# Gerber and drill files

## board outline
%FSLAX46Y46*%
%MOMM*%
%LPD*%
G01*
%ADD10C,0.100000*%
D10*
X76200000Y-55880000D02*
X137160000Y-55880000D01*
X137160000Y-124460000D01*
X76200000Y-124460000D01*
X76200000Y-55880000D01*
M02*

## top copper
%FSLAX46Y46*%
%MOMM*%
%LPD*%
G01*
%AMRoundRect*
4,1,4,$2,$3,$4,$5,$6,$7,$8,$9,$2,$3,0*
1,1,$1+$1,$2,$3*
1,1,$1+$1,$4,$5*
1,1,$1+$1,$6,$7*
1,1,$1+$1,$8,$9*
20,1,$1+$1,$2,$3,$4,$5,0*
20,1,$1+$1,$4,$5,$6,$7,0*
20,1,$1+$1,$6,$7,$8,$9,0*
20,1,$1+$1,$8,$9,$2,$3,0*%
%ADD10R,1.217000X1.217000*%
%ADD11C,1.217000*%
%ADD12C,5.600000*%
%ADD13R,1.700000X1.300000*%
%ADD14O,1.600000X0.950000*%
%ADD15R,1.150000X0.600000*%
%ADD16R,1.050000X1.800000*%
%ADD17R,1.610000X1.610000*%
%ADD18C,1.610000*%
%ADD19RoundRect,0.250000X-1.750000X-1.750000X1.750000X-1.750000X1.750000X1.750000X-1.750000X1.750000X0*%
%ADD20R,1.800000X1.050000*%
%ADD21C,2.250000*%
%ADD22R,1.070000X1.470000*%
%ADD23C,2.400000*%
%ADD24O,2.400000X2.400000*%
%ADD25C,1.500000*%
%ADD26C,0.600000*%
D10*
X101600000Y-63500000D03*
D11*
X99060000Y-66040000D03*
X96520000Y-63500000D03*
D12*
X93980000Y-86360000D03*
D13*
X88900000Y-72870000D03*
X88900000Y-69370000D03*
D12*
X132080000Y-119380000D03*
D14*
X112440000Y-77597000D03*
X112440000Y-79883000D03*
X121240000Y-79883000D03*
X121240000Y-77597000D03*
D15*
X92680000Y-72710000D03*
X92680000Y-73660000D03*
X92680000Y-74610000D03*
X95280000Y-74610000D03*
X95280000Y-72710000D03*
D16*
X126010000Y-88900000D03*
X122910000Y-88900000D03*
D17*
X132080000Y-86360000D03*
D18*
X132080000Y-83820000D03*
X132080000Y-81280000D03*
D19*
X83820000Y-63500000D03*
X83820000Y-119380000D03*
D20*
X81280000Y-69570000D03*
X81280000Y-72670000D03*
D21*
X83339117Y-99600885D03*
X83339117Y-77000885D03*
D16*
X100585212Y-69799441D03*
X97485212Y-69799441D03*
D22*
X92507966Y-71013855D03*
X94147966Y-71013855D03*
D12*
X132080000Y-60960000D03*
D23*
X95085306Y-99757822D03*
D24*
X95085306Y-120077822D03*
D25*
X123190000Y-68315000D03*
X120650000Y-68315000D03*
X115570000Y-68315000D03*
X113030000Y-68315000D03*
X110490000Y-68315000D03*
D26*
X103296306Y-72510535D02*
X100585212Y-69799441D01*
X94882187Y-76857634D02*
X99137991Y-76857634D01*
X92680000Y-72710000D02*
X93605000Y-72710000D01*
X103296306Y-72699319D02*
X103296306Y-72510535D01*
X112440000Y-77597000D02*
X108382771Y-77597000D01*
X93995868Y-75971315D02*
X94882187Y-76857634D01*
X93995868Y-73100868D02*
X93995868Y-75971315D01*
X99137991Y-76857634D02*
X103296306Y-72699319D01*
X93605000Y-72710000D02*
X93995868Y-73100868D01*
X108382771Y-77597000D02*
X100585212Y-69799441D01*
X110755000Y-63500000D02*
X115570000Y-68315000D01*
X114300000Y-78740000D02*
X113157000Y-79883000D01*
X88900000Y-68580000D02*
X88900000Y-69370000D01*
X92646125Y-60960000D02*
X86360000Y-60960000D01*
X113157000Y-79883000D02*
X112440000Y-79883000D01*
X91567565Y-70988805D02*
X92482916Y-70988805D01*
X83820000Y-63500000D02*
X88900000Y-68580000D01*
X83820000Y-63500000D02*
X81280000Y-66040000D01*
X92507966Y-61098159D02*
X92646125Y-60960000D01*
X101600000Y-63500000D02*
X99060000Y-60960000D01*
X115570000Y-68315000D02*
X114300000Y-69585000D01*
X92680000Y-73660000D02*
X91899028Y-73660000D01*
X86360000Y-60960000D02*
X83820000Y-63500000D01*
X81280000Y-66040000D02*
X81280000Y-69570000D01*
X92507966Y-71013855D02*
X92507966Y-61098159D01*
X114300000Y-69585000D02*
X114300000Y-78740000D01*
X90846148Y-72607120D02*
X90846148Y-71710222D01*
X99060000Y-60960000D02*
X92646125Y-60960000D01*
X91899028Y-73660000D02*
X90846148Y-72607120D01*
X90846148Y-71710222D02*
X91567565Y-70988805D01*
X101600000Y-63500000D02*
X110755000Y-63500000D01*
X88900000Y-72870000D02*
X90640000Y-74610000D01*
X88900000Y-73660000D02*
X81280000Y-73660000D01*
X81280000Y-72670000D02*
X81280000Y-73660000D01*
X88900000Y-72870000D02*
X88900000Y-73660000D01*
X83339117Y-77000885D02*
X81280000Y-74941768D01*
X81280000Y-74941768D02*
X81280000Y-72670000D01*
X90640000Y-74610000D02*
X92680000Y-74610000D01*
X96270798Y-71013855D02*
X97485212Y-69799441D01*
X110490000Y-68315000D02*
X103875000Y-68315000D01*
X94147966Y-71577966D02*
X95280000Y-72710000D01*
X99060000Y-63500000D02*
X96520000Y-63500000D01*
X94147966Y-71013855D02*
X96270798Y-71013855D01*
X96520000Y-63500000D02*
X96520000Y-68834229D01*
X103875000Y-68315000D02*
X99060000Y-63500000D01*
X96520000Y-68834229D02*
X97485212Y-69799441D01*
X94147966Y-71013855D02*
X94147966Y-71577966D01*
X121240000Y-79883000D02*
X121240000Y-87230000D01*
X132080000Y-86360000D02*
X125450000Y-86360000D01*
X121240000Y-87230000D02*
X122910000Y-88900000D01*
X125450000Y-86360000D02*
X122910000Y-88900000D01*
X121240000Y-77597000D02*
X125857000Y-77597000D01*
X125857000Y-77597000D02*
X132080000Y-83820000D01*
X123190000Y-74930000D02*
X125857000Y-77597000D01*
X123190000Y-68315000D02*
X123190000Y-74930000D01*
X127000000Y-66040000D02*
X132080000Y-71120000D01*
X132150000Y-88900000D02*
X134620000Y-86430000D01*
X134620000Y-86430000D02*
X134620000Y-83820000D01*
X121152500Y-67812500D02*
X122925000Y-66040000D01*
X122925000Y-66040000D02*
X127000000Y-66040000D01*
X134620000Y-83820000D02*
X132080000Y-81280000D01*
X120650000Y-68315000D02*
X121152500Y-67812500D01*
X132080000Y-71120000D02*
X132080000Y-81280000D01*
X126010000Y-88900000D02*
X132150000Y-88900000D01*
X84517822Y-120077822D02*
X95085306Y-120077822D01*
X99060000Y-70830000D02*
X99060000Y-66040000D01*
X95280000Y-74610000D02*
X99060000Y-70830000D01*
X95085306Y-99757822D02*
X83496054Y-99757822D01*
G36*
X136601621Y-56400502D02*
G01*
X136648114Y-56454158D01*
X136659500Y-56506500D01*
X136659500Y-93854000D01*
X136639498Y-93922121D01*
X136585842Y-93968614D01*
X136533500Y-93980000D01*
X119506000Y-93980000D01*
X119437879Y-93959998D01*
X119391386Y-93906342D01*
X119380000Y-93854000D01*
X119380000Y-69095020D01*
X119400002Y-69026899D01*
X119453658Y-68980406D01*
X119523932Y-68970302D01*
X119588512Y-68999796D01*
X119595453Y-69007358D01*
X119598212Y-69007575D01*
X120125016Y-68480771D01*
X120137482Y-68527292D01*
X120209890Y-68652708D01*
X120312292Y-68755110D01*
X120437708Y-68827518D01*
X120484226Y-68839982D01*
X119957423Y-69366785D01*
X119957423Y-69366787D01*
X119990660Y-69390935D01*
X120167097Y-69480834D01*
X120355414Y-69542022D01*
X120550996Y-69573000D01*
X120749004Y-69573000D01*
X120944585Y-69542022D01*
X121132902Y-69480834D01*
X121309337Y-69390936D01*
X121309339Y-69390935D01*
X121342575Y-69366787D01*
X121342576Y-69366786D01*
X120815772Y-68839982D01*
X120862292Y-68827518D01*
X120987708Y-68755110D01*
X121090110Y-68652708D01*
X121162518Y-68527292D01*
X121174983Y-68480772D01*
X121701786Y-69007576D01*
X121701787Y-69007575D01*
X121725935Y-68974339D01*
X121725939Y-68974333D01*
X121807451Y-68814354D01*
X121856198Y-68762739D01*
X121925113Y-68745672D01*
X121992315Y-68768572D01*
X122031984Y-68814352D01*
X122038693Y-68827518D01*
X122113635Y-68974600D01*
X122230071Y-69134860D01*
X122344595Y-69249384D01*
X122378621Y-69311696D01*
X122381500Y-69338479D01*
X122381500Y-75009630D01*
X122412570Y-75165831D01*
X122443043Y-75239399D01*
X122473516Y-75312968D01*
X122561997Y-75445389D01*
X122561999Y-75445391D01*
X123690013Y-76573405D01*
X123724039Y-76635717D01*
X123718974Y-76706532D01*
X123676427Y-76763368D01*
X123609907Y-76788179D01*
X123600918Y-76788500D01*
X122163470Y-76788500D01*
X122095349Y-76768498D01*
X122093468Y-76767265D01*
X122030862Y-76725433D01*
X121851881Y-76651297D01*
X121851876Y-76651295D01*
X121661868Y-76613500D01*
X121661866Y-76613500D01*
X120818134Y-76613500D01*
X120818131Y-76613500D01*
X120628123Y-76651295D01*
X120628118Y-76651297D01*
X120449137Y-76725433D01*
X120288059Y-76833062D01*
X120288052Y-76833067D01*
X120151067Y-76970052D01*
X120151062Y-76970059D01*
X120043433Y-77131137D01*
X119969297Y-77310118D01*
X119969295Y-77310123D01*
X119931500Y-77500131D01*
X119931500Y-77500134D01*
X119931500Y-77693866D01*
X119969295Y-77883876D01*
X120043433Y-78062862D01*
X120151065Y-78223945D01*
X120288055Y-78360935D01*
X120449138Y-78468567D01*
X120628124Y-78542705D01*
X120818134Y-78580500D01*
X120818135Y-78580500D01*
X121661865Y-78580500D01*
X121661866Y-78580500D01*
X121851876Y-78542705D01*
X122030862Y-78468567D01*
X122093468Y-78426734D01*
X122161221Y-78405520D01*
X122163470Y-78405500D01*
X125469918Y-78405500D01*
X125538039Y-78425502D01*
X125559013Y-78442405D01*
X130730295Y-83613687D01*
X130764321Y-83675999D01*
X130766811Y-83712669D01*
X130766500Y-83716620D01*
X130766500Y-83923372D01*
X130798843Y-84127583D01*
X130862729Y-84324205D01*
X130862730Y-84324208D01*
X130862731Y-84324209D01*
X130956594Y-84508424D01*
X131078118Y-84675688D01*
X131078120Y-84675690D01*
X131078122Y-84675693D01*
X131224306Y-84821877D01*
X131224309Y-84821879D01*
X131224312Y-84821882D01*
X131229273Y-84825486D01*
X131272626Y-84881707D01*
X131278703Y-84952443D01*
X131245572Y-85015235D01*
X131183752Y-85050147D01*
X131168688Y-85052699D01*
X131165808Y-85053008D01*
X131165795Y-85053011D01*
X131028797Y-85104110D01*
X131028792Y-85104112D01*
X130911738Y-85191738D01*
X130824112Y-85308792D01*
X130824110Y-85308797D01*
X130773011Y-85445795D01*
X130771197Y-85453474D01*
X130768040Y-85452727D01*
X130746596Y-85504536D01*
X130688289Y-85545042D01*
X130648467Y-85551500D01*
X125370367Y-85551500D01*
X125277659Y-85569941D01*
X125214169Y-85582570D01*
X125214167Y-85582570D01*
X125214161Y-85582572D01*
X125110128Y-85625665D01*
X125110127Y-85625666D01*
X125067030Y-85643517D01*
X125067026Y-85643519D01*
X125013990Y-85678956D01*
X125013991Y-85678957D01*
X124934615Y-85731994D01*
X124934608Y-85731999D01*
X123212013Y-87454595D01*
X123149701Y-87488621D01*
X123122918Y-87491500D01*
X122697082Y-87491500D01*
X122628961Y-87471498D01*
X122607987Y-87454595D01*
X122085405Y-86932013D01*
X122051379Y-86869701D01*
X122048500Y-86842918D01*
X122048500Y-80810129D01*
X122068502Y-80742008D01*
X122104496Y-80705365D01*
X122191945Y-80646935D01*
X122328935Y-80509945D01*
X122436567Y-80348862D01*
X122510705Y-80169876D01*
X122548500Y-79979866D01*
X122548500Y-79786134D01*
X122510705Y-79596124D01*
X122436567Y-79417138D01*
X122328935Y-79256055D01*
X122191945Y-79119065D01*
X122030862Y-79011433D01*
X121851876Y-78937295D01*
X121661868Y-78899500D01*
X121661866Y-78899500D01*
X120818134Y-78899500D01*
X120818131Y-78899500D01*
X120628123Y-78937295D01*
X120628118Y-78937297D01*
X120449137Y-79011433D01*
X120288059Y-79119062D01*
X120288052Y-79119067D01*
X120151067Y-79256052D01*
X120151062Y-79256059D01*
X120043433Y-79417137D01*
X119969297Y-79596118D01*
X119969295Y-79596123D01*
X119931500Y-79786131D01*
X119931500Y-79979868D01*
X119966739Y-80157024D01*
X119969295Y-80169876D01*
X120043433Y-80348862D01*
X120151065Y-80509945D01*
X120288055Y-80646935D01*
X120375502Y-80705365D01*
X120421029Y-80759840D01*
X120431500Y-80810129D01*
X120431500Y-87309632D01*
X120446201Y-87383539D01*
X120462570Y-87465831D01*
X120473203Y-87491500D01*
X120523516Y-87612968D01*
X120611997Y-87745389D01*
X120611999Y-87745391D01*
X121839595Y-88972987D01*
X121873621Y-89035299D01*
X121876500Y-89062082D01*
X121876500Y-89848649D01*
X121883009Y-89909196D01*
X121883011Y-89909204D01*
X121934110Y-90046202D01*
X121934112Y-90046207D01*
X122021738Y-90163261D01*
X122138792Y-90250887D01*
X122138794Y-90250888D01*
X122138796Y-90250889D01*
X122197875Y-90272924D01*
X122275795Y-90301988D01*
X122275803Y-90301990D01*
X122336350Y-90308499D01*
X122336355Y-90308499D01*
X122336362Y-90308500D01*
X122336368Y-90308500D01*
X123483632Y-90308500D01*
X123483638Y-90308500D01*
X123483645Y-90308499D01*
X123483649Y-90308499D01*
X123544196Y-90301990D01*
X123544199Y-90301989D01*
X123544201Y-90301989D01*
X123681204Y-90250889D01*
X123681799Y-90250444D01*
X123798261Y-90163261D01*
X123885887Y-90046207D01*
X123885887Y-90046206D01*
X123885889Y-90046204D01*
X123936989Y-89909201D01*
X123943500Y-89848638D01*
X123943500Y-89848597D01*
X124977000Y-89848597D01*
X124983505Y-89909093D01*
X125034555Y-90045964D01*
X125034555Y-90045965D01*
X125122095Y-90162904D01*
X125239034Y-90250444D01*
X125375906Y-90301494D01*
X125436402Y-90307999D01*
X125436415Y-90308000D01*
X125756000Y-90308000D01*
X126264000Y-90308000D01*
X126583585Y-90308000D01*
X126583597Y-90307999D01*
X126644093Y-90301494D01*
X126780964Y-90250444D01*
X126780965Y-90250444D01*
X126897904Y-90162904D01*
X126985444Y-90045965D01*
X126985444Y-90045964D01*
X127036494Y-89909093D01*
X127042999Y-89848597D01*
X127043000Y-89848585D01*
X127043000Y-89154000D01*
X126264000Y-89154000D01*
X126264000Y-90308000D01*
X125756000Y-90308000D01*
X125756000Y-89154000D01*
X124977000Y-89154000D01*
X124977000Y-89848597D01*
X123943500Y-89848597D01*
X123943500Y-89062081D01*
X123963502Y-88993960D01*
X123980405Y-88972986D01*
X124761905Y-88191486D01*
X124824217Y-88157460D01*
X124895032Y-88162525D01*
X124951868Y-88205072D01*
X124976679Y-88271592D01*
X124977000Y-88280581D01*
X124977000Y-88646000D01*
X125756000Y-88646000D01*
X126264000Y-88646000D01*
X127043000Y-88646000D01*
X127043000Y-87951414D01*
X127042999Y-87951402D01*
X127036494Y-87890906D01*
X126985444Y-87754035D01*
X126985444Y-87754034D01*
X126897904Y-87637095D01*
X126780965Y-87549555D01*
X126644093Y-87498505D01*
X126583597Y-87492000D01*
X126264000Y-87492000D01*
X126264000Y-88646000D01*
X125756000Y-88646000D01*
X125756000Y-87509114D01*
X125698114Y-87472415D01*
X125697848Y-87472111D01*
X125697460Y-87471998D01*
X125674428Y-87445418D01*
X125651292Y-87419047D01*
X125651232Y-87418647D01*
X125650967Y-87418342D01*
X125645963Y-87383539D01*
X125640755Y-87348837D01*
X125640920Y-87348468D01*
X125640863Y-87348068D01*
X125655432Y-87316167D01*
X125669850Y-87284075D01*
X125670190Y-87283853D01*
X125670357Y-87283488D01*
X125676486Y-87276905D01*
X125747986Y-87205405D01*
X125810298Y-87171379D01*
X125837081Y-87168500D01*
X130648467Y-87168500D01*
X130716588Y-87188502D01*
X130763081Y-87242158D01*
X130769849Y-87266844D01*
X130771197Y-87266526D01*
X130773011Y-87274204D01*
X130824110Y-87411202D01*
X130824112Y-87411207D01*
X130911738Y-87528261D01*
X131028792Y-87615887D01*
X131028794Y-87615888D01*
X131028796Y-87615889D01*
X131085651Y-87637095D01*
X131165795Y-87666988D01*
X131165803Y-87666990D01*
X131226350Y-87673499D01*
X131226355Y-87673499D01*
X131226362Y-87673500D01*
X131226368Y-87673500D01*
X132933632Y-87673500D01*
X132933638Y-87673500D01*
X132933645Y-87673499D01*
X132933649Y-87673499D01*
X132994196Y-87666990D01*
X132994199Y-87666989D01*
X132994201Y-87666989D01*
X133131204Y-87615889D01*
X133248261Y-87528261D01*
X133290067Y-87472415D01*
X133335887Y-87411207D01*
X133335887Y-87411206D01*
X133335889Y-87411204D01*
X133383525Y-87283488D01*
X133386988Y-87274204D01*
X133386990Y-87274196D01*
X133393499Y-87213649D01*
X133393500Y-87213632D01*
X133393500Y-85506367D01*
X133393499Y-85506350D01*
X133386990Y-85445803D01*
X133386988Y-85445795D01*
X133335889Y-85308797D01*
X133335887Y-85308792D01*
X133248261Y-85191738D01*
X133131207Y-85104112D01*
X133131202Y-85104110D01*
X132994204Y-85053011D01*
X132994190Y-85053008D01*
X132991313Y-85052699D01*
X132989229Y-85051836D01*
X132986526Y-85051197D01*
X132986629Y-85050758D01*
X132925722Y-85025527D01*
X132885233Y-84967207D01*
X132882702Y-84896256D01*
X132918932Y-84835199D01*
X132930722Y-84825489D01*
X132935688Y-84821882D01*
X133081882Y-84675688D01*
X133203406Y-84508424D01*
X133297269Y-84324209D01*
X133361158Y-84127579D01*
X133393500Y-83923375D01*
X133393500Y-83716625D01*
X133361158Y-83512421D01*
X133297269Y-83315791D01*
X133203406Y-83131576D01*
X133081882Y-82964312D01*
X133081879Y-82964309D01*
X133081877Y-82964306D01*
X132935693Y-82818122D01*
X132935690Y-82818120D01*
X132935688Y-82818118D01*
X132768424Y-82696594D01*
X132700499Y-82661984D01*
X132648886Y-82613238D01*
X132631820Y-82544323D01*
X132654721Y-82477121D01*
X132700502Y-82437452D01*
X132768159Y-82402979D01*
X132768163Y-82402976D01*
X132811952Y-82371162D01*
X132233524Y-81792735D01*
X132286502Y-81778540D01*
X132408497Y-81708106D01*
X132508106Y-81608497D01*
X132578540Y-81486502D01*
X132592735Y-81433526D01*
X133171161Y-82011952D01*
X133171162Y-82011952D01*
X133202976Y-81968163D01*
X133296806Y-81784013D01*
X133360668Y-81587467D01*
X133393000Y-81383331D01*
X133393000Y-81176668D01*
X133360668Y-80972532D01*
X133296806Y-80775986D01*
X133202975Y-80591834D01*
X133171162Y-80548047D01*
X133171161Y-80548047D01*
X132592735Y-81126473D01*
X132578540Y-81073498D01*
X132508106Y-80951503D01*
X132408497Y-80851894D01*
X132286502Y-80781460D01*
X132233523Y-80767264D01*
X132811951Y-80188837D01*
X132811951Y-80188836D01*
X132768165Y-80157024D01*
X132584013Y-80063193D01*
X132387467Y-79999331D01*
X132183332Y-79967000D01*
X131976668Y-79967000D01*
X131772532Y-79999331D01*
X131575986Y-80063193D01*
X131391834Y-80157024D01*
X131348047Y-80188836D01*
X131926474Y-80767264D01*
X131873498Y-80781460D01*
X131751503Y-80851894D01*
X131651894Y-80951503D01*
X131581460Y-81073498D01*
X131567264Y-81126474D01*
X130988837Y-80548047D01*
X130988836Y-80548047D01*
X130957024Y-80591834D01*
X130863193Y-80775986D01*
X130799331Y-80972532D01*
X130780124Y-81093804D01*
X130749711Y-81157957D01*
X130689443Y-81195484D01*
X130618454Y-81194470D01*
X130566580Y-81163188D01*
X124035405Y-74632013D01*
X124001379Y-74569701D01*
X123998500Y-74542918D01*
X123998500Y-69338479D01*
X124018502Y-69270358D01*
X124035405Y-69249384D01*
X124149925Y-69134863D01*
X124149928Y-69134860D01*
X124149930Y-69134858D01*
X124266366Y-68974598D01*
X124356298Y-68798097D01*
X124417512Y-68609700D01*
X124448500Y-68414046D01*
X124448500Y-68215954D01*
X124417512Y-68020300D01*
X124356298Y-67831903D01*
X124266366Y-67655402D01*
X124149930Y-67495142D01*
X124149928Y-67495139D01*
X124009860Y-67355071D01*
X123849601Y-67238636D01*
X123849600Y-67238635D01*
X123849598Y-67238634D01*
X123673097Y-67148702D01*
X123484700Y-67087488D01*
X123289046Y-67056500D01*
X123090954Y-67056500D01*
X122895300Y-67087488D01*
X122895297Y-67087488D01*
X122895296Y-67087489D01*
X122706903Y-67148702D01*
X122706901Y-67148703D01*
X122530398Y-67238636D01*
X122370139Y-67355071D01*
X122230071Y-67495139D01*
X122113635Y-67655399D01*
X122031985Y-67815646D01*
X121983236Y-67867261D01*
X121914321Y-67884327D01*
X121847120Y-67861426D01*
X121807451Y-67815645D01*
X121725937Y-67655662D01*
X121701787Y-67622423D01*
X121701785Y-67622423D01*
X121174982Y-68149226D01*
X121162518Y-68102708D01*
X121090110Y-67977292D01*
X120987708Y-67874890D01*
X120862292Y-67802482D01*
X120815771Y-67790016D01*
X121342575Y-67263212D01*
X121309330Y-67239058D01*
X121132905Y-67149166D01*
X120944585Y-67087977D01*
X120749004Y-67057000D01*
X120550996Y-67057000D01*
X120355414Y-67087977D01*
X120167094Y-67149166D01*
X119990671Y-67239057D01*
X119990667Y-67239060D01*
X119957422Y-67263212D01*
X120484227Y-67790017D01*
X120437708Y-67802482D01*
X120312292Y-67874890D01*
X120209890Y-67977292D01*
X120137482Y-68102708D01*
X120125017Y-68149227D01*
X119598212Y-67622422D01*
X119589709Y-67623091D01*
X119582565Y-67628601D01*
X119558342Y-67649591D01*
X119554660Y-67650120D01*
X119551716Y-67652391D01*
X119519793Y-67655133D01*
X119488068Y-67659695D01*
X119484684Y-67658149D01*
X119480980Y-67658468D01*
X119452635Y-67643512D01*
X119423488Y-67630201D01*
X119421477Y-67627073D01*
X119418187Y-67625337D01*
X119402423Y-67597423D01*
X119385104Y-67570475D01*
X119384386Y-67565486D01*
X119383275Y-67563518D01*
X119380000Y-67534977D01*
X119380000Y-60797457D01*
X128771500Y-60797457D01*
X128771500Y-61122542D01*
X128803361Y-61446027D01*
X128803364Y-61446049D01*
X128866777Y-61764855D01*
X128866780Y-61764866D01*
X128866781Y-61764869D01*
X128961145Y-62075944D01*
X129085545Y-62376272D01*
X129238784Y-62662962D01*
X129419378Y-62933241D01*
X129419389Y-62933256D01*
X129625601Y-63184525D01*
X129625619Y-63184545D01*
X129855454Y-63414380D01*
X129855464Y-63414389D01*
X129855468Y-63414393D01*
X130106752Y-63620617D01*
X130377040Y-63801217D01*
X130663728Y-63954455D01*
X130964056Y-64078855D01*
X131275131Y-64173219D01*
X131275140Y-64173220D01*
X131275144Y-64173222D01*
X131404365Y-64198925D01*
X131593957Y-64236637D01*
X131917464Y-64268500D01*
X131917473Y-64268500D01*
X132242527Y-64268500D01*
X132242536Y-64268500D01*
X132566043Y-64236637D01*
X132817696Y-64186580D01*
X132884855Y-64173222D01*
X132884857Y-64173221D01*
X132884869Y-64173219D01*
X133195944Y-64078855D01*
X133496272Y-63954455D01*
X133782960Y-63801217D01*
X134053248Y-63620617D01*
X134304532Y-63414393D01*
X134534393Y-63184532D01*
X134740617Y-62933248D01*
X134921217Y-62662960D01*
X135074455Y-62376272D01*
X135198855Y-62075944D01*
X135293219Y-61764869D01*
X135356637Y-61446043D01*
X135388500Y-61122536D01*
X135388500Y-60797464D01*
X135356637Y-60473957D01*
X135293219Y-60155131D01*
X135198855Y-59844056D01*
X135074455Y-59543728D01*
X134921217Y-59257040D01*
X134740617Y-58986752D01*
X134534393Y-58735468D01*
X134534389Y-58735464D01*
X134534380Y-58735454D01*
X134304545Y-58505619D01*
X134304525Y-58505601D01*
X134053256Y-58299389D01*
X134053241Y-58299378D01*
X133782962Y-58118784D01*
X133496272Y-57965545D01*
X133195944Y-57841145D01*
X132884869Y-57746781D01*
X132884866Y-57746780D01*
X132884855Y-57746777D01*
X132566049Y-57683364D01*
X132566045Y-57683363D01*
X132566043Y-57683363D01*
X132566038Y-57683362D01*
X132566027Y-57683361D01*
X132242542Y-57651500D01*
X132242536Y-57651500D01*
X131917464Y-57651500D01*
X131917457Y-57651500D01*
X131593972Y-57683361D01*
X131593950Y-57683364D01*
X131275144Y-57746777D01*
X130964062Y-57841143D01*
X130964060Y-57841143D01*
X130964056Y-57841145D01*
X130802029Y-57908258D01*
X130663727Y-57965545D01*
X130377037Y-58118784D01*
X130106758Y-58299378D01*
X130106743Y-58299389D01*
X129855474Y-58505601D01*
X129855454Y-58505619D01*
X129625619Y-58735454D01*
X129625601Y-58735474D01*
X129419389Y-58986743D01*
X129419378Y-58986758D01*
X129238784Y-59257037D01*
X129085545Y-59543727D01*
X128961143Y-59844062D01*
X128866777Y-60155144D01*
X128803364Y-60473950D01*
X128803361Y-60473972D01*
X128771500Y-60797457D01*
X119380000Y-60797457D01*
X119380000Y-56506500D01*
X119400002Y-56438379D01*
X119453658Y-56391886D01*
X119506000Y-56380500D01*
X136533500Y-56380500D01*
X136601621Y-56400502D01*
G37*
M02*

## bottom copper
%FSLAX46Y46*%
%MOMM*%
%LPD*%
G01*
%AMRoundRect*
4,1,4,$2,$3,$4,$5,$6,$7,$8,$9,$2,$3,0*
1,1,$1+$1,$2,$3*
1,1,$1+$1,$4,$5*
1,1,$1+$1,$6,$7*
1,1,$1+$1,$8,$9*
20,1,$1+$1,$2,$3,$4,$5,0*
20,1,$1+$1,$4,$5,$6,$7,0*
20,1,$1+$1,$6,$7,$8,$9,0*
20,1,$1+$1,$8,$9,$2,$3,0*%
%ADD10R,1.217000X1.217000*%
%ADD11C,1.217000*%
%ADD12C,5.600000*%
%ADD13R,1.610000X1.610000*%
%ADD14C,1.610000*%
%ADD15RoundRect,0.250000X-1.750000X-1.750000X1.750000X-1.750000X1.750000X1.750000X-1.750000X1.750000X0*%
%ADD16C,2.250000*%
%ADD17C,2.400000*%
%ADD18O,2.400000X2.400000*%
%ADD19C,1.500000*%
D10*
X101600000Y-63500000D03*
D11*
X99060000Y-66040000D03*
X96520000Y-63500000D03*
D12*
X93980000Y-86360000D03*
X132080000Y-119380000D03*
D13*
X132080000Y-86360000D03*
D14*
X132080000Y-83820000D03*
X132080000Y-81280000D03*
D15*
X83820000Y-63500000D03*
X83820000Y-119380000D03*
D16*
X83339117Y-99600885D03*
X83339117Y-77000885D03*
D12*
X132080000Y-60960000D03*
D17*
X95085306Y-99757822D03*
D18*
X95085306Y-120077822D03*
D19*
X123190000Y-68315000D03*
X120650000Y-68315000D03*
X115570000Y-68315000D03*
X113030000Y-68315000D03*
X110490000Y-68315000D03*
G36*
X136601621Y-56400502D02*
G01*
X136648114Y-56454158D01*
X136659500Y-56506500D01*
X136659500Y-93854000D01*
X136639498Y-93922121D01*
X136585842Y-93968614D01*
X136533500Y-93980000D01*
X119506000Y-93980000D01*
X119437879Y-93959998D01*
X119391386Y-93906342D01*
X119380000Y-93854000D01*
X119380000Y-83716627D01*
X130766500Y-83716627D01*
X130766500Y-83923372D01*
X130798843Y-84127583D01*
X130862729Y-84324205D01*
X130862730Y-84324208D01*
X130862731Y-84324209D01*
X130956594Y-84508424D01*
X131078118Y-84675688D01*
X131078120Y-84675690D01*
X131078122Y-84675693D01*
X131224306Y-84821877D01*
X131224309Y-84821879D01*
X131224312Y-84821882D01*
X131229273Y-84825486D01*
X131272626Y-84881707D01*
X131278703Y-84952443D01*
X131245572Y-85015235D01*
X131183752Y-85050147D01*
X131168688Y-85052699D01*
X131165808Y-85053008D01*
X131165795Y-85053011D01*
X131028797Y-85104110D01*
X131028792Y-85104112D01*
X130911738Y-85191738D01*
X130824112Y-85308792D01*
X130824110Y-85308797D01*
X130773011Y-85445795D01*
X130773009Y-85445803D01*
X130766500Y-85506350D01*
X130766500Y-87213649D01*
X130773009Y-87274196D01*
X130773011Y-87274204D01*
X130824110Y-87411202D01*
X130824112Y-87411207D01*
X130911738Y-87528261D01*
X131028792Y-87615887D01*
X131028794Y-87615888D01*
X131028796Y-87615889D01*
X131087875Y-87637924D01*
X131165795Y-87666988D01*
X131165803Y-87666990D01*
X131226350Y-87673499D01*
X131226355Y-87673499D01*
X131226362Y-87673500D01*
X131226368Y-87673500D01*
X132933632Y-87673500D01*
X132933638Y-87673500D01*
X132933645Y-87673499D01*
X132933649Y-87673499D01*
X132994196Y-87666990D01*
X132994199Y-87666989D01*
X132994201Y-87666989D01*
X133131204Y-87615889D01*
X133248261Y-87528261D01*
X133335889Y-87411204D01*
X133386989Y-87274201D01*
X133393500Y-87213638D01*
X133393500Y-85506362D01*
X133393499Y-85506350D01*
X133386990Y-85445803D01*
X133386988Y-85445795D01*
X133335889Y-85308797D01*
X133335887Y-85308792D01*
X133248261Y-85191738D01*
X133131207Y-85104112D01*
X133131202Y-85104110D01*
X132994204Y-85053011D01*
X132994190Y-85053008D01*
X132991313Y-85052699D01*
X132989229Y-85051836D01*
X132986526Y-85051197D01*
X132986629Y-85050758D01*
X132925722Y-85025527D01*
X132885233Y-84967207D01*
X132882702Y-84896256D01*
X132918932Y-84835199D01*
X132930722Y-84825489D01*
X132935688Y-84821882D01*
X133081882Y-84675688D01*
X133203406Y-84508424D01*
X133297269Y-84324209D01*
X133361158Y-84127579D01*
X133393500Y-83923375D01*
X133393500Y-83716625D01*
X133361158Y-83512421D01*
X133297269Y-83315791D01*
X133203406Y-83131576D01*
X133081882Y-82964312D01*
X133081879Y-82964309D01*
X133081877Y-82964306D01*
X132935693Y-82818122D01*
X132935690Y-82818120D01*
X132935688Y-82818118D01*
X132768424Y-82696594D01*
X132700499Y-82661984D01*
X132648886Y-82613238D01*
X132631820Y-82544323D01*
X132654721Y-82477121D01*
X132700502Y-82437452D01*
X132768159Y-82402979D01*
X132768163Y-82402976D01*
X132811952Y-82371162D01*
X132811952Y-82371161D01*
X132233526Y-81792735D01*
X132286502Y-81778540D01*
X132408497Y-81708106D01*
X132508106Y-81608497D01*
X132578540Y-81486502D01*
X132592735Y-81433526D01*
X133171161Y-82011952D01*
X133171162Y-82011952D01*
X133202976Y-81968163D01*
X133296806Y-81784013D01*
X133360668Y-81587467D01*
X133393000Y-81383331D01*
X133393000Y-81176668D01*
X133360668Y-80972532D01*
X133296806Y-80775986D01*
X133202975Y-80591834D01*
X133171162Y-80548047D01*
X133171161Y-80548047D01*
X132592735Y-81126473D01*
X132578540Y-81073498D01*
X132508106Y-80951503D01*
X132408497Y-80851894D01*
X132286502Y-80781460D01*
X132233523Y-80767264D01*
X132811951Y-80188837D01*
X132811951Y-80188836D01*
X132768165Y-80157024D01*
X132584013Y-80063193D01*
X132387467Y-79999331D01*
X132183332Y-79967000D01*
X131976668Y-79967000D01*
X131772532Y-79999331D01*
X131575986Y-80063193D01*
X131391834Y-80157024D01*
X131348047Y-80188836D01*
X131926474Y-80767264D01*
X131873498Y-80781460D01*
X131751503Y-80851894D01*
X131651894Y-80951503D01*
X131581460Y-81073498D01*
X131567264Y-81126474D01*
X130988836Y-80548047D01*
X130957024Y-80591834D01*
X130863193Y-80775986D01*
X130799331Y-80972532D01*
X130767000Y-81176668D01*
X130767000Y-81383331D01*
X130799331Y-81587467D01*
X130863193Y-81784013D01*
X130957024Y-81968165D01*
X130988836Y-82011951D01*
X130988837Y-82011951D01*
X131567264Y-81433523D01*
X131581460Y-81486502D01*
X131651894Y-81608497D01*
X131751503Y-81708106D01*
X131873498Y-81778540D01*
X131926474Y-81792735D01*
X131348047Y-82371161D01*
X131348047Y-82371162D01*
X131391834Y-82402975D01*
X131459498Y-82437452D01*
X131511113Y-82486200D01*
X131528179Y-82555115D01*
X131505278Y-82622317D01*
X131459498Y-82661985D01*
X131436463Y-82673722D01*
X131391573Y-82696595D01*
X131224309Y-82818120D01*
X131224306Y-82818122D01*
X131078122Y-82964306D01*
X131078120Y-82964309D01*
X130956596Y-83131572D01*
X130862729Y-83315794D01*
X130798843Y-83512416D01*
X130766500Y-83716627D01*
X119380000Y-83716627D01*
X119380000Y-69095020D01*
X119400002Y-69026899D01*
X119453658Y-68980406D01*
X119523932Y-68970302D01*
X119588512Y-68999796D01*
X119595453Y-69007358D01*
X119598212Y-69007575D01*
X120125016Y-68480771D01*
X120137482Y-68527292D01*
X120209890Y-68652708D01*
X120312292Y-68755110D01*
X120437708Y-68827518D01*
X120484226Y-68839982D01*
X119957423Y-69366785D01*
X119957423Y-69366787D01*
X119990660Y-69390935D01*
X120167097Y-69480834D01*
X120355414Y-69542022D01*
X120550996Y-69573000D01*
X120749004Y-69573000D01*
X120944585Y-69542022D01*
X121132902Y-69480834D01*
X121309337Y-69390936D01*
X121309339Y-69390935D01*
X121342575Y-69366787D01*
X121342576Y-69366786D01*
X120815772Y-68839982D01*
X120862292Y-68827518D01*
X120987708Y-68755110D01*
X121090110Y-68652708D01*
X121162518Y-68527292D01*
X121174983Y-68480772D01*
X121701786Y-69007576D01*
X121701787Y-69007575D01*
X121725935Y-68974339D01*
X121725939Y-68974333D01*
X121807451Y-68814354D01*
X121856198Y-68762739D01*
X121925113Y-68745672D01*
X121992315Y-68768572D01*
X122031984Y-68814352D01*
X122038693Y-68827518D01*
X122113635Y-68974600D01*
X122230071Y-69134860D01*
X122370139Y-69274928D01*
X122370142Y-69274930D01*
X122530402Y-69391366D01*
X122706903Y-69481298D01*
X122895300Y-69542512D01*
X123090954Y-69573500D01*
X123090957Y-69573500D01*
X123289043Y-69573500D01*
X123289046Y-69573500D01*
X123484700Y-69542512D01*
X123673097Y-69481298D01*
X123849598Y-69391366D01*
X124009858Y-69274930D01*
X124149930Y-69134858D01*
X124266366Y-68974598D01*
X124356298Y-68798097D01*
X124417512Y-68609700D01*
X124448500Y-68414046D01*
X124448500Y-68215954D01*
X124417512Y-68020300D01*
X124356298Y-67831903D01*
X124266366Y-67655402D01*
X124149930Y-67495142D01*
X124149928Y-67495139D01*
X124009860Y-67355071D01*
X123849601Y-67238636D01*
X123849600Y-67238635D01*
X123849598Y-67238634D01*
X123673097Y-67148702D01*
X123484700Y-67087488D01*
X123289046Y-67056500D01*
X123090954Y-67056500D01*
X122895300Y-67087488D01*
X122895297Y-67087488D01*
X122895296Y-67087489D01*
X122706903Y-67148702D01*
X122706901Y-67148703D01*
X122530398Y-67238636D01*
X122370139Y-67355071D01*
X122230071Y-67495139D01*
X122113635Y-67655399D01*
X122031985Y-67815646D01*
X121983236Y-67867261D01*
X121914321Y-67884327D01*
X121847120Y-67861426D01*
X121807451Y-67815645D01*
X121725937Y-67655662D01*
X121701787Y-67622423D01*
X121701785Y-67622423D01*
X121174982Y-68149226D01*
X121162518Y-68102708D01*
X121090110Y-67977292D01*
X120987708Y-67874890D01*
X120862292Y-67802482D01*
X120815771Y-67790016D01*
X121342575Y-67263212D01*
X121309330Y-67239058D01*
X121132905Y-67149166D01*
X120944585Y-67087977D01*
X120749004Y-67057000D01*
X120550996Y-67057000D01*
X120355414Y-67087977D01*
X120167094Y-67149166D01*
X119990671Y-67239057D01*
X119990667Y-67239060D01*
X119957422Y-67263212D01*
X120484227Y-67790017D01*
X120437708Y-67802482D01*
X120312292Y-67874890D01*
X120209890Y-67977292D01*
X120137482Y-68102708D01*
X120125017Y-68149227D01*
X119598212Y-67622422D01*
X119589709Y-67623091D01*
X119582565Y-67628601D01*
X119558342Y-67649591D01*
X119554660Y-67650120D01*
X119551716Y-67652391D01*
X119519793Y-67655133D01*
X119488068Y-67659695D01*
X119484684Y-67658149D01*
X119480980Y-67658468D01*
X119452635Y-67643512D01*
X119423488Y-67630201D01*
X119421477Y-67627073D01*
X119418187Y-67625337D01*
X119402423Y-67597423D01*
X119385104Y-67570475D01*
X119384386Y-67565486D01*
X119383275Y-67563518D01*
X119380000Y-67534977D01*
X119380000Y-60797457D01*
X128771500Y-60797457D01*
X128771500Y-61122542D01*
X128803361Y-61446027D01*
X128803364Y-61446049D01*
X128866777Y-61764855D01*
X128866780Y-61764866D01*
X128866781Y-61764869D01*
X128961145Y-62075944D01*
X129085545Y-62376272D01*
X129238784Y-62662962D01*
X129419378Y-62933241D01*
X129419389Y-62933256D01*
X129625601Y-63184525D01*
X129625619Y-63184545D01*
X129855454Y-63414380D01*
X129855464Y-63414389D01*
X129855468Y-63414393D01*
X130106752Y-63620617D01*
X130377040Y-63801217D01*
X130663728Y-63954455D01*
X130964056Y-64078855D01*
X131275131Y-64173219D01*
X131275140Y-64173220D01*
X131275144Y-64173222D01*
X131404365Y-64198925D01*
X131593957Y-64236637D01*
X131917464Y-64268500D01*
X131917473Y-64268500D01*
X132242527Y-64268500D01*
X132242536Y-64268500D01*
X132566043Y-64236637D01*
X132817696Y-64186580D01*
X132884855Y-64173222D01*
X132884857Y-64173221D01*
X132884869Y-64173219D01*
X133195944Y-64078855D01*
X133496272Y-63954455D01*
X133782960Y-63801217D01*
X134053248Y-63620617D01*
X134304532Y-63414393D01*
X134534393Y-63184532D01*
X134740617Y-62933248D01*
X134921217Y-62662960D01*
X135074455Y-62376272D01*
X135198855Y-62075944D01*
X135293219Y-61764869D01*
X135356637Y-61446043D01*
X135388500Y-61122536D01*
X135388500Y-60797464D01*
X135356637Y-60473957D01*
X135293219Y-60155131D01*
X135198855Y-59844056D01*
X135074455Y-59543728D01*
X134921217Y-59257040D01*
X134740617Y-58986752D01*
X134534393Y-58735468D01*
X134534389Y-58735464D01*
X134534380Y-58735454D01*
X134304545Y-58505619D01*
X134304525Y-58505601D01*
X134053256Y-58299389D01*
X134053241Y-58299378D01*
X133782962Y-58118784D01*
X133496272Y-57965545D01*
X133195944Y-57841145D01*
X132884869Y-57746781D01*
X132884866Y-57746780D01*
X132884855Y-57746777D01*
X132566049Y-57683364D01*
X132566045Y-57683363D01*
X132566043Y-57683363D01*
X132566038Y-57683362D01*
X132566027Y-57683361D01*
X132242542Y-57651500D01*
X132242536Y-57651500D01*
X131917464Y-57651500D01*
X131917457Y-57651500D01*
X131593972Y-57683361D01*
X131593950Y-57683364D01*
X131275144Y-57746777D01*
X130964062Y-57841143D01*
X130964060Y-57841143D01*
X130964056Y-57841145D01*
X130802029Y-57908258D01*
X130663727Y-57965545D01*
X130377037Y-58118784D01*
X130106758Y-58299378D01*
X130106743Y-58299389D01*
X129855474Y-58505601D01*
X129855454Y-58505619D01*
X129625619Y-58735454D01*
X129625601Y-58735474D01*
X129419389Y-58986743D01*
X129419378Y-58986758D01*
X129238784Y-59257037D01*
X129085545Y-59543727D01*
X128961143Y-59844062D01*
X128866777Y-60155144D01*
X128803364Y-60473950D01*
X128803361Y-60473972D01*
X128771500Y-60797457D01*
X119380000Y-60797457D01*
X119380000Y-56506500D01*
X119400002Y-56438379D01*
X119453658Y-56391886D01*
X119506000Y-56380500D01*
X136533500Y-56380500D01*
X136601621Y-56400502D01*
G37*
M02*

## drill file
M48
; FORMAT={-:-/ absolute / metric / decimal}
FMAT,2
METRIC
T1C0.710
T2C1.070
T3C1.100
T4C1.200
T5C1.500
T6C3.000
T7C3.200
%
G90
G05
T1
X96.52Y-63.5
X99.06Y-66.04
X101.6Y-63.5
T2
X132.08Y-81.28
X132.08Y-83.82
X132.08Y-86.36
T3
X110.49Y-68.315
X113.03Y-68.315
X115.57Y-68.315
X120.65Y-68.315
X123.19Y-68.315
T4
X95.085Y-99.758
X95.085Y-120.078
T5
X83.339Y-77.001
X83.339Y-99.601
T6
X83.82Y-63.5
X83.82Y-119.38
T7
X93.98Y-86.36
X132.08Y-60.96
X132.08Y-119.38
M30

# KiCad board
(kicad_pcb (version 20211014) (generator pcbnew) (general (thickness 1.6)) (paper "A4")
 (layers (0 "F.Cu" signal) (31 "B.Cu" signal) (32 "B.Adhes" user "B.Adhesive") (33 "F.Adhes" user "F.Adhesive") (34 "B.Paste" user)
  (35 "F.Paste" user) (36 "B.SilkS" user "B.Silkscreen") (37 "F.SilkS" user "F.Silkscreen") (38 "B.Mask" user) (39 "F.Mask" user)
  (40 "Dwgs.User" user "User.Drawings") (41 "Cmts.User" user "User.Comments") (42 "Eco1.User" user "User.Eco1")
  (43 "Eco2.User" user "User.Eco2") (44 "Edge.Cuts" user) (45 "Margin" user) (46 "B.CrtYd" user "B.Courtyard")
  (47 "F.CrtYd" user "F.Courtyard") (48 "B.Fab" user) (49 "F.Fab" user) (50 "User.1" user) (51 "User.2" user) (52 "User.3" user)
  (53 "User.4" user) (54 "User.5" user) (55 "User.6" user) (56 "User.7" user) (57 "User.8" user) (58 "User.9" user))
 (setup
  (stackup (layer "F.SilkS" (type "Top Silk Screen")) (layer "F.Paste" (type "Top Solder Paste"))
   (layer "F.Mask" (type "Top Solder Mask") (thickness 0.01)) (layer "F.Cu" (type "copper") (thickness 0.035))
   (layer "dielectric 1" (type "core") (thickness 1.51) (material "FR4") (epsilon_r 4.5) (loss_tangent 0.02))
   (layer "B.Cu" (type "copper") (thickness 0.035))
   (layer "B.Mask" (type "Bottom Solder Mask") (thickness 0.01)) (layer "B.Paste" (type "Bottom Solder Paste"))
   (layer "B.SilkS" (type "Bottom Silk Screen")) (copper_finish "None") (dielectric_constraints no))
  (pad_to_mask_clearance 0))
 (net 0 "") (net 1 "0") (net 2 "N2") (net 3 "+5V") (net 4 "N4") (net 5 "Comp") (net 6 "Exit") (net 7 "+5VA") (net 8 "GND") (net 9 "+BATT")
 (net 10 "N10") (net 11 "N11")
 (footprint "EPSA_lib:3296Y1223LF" (layer "F.Cu") (at 101.6 63.5 90)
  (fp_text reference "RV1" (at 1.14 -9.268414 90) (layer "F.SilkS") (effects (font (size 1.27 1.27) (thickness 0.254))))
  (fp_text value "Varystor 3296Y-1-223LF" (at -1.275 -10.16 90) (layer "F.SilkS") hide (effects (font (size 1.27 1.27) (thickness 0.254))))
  (pad "1" thru_hole rect (at 0 0 90) (size 1.217 1.217) (drill 0.71) (layers *.Cu *.Mask) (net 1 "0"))
  (pad "2" thru_hole circle (at -2.54 -2.54 90) (size 1.217 1.217) (drill 0.71) (layers *.Cu *.Mask) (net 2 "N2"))
  (pad "3" thru_hole circle (at 0 -5.08 90) (size 1.217 1.217) (drill 0.71) (layers *.Cu *.Mask) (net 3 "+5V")))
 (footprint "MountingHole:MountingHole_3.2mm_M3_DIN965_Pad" (layer "F.Cu") (at 93.98 86.36)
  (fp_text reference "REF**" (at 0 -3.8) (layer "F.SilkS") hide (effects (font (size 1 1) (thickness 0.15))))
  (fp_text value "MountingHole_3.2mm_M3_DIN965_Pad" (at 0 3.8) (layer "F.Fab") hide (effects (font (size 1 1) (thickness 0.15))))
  (pad "1" thru_hole circle (at 0 0) (size 5.6 5.6) (drill 3.2) (layers *.Cu *.Mask)))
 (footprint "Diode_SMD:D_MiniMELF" (layer "F.Cu") (at 88.9 71.12 90)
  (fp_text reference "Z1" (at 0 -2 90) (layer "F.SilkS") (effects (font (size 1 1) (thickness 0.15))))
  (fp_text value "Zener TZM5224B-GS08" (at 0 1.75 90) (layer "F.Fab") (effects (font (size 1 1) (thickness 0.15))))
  (pad "1" smd rect (at -1.75 0 90) (size 1.3 1.7) (layers "F.Cu" "F.Paste" "F.Mask") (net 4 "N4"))
  (pad "2" smd rect (at 1.75 0 90) (size 1.3 1.7) (layers "F.Cu" "F.Paste" "F.Mask") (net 1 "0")))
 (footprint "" (layer "F.Cu") (at 132.08 119.38)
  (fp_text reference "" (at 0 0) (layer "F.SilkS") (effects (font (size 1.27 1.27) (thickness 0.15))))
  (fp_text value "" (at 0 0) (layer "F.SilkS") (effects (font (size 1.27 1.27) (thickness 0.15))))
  (pad "1" thru_hole circle (at 0 0) (size 5.6 5.6) (drill 3.2) (layers *.Cu *.Mask)))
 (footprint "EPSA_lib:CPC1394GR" (layer "F.Cu") (at 116.84 78.74 -90)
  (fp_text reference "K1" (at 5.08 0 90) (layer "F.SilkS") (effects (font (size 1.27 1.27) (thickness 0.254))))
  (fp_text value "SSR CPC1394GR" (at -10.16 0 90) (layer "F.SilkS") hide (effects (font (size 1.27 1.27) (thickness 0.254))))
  (pad "1" smd oval (at -1.143 4.4 270) (size 0.95 1.6) (layers "F.Cu" "F.Paste" "F.Mask") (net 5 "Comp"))
  (pad "2" smd oval (at 1.143 4.4 270) (size 0.95 1.6) (layers "F.Cu" "F.Paste" "F.Mask") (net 1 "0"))
  (pad "3" smd oval (at 1.143 -4.4 270) (size 0.95 1.6) (layers "F.Cu" "F.Paste" "F.Mask") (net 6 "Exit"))
  (pad "4" smd oval (at -1.143 -4.4 270) (size 0.95 1.6) (layers "F.Cu" "F.Paste" "F.Mask") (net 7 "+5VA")))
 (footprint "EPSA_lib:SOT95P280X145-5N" (layer "F.Cu") (at 93.98 73.66)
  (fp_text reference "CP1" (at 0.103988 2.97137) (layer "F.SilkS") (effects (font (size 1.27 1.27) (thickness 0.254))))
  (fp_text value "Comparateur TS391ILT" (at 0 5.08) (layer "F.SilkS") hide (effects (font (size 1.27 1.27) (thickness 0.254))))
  (pad "1" smd rect (at -1.3 -0.95 90) (size 0.6 1.15) (layers "F.Cu" "F.Paste" "F.Mask") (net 5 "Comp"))
  (pad "2" smd rect (at -1.3 0 90) (size 0.6 1.15) (layers "F.Cu" "F.Paste" "F.Mask") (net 1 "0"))
  (pad "3" smd rect (at -1.3 0.95 90) (size 0.6 1.15) (layers "F.Cu" "F.Paste" "F.Mask") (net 4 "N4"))
  (pad "4" smd rect (at 1.3 0.95 90) (size 0.6 1.15) (layers "F.Cu" "F.Paste" "F.Mask") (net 2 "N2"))
  (pad "5" smd rect (at 1.3 -0.95 90) (size 0.6 1.15) (layers "F.Cu" "F.Paste" "F.Mask") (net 3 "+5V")))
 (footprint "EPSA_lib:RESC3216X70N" (layer "F.Cu") (at 124.46 88.9 180)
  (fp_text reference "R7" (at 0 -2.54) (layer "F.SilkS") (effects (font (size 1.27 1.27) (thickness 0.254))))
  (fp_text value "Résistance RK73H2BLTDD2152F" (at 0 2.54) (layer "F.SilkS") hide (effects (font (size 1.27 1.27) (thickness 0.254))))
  (pad "1" smd rect (at -1.55 0 180) (size 1.05 1.8) (layers "F.Cu" "F.Paste" "F.Mask") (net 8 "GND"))
  (pad "2" smd rect (at 1.55 0 180) (size 1.05 1.8) (layers "F.Cu" "F.Paste" "F.Mask") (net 6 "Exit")))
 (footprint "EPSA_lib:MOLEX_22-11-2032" (layer "F.Cu") (at 132.08 86.36 90)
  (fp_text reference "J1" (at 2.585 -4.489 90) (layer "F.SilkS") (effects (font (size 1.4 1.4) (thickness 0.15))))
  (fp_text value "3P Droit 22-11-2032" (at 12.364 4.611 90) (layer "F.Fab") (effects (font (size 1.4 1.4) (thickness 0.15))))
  (pad "1" thru_hole rect (at 0 0 90) (size 1.61 1.61) (drill 1.07) (layers *.Cu *.Mask) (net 6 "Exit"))
  (pad "2" thru_hole circle (at 2.54 0 90) (size 1.61 1.61) (drill 1.07) (layers *.Cu *.Mask) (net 7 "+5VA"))
  (pad "3" thru_hole circle (at 5.08 0 90) (size 1.61 1.61) (drill 1.07) (layers *.Cu *.Mask) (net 8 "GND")))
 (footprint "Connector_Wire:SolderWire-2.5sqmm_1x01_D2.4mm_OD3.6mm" (layer "F.Cu") (at 83.82 63.5)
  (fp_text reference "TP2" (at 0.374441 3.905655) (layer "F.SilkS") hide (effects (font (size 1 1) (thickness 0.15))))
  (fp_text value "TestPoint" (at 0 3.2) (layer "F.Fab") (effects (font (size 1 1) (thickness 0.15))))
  (pad "1" thru_hole roundrect (at 0 0) (size 4 4) (drill 3) (layers *.Cu *.Mask) (roundrect_rratio 0.0625) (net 1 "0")))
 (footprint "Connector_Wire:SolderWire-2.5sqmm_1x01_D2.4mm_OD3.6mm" (layer "F.Cu") (at 83.82 119.38)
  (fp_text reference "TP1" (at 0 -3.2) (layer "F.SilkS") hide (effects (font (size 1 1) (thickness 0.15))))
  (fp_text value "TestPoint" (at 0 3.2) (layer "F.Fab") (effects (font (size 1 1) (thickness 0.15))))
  (pad "1" thru_hole roundrect (at 0 0) (size 4 4) (drill 3) (layers *.Cu *.Mask) (roundrect_rratio 0.0625) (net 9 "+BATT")))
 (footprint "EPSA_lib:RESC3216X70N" (layer "F.Cu") (at 81.28 71.12 -90)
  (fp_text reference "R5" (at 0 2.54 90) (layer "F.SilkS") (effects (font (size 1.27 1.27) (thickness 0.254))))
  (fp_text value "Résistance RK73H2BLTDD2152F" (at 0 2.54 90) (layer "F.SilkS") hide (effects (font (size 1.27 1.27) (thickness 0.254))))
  (pad "1" smd rect (at -1.55 0 270) (size 1.05 1.8) (layers "F.Cu" "F.Paste" "F.Mask") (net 1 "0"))
  (pad "2" smd rect (at 1.55 0 270) (size 1.05 1.8) (layers "F.Cu" "F.Paste" "F.Mask") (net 4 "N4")))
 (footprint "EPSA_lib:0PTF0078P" (layer "F.Cu") (at 83.339117 88.300885 90)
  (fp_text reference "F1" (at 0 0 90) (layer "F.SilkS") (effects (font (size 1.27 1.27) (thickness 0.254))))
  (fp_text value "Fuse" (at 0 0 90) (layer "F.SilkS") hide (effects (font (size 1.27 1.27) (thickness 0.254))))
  (pad "1" thru_hole circle locked (at -11.3 0 90) (size 2.25 2.25) (drill 1.5) (layers *.Cu *.Mask) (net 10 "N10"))
  (pad "2" thru_hole circle locked (at 11.3 0 90) (size 2.25 2.25) (drill 1.5) (layers *.Cu *.Mask) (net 4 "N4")))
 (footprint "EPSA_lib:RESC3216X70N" (layer "F.Cu") (at 99.035212 69.799441 180)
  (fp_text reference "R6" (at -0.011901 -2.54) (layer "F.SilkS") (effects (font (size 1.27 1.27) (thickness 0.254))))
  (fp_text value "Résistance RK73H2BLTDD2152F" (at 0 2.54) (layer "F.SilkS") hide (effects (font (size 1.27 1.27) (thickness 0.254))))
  (pad "1" smd rect (at -1.55 0 180) (size 1.05 1.8) (layers "F.Cu" "F.Paste" "F.Mask") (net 5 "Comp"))
  (pad "2" smd rect (at 1.55 0 180) (size 1.05 1.8) (layers "F.Cu" "F.Paste" "F.Mask") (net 3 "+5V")))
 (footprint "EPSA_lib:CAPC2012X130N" (layer "F.Cu") (at 93.327966 71.013855)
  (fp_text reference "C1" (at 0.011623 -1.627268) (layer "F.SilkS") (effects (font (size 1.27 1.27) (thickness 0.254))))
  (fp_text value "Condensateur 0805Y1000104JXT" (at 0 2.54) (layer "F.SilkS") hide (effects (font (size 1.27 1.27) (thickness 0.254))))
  (pad "1" smd rect (at -0.82 0) (size 1.07 1.47) (layers "F.Cu" "F.Paste" "F.Mask") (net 1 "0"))
  (pad "2" smd rect (at 0.82 0) (size 1.07 1.47) (layers "F.Cu" "F.Paste" "F.Mask") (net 3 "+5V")))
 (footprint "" (layer "F.Cu") (at 132.08 60.96)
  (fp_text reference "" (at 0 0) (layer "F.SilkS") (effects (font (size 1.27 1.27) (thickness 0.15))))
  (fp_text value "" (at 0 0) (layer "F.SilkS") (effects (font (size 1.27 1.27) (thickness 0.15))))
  (pad "1" thru_hole circle (at 0 0) (size 5.6 5.6) (drill 3.2) (layers *.Cu *.Mask)))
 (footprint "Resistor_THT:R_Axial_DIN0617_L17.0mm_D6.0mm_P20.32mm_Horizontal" (layer "F.Cu") (at 95.085306 99.757822 -90)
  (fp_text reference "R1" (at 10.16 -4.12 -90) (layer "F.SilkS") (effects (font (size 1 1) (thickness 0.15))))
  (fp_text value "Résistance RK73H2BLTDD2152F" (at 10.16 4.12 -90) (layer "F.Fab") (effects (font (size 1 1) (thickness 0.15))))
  (pad "1" thru_hole circle (at 0 0 270) (size 2.4 2.4) (drill 1.2) (layers *.Cu *.Mask) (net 10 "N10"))
  (pad "2" thru_hole oval (at 20.32 0 270) (size 2.4 2.4) (drill 1.2) (layers *.Cu *.Mask) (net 9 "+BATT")))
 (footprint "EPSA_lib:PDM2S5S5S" (layer "F.Cu") (at 123.19 68.315 180)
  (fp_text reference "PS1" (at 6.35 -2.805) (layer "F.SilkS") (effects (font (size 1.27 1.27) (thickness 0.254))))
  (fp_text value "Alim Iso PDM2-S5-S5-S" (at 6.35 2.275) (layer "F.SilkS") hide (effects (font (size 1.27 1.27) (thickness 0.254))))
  (pad "1" thru_hole circle (at 0 0 180) (size 1.5 1.5) (drill 1.1) (layers *.Cu *.Mask) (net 7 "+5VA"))
  (pad "2" thru_hole circle (at 2.54 0 180) (size 1.5 1.5) (drill 1.1) (layers *.Cu *.Mask) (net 8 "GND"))
  (pad "4" thru_hole circle (at 7.62 0 180) (size 1.5 1.5) (drill 1.1) (layers *.Cu *.Mask) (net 1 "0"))
  (pad "5" thru_hole circle (at 10.16 0 180) (size 1.5 1.5) (drill 1.1) (layers *.Cu *.Mask) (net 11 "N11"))
  (pad "6" thru_hole circle (at 12.7 0 180) (size 1.5 1.5) (drill 1.1) (layers *.Cu *.Mask) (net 3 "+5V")))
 (gr_rect (start 137.16 55.88) (end 76.2 124.46) (layer "Edge.Cuts") (width 0.1) (fill none))
 (segment (start 103.296306 72.510535) (end 100.585212 69.799441) (width 0.6) (layer "F.Cu") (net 5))
 (segment (start 94.882187 76.857634) (end 99.137991 76.857634) (width 0.6) (layer "F.Cu") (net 5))
 (segment (start 92.68 72.71) (end 93.605 72.71) (width 0.6) (layer "F.Cu") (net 5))
 (segment (start 103.296306 72.699319) (end 103.296306 72.510535) (width 0.6) (layer "F.Cu") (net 5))
 (segment (start 112.44 77.597) (end 108.382771 77.597) (width 0.6) (layer "F.Cu") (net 5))
 (segment (start 93.995868 75.971315) (end 94.882187 76.857634) (width 0.6) (layer "F.Cu") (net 5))
 (segment (start 93.995868 73.100868) (end 93.995868 75.971315) (width 0.6) (layer "F.Cu") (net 5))
 (segment (start 99.137991 76.857634) (end 103.296306 72.699319) (width 0.6) (layer "F.Cu") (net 5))
 (segment (start 93.605 72.71) (end 93.995868 73.100868) (width 0.6) (layer "F.Cu") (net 5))
 (segment (start 108.382771 77.597) (end 100.585212 69.799441) (width 0.6) (layer "F.Cu") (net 5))
 (segment (start 110.755 63.5) (end 115.57 68.315) (width 0.6) (layer "F.Cu") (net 1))
 (segment (start 114.3 78.74) (end 113.157 79.883) (width 0.6) (layer "F.Cu") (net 1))
 (segment (start 88.9 68.58) (end 88.9 69.37) (width 0.6) (layer "F.Cu") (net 1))
 (segment (start 92.646125 60.96) (end 86.36 60.96) (width 0.6) (layer "F.Cu") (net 1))
 (segment (start 113.157 79.883) (end 112.44 79.883) (width 0.6) (layer "F.Cu") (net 1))
 (segment (start 91.567565 70.988805) (end 92.482916 70.988805) (width 0.6) (layer "F.Cu") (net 1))
 (segment (start 83.82 63.5) (end 88.9 68.58) (width 0.6) (layer "F.Cu") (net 1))
 (segment (start 83.82 63.5) (end 81.28 66.04) (width 0.6) (layer "F.Cu") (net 1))
 (segment (start 92.507966 61.098159) (end 92.646125 60.96) (width 0.6) (layer "F.Cu") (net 1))
 (segment (start 101.6 63.5) (end 99.06 60.96) (width 0.6) (layer "F.Cu") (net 1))
 (segment (start 115.57 68.315) (end 114.3 69.585) (width 0.6) (layer "F.Cu") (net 1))
 (segment (start 92.68 73.66) (end 91.899028 73.66) (width 0.6) (layer "F.Cu") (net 1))
 (segment (start 86.36 60.96) (end 83.82 63.5) (width 0.6) (layer "F.Cu") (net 1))
 (segment (start 81.28 66.04) (end 81.28 69.57) (width 0.6) (layer "F.Cu") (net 1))
 (segment (start 92.507966 71.013855) (end 92.507966 61.098159) (width 0.6) (layer "F.Cu") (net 1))
 (segment (start 114.3 69.585) (end 114.3 78.74) (width 0.6) (layer "F.Cu") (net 1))
 (segment (start 90.846148 72.60712) (end 90.846148 71.710222) (width 0.6) (layer "F.Cu") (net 1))
 (segment (start 99.06 60.96) (end 92.646125 60.96) (width 0.6) (layer "F.Cu") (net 1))
 (segment (start 91.899028 73.66) (end 90.846148 72.60712) (width 0.6) (layer "F.Cu") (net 1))
 (segment (start 90.846148 71.710222) (end 91.567565 70.988805) (width 0.6) (layer "F.Cu") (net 1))
 (segment (start 101.6 63.5) (end 110.755 63.5) (width 0.6) (layer "F.Cu") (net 1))
 (segment (start 88.9 72.87) (end 90.64 74.61) (width 0.6) (layer "F.Cu") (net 4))
 (segment (start 88.9 73.66) (end 81.28 73.66) (width 0.6) (layer "F.Cu") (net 4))
 (segment (start 81.28 72.67) (end 81.28 73.66) (width 0.6) (layer "F.Cu") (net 4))
 (segment (start 88.9 72.87) (end 88.9 73.66) (width 0.6) (layer "F.Cu") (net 4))
 (segment (start 83.339117 77.000885) (end 81.28 74.941768) (width 0.6) (layer "F.Cu") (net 4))
 (segment (start 81.28 74.941768) (end 81.28 72.67) (width 0.6) (layer "F.Cu") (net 4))
 (segment (start 90.64 74.61) (end 92.68 74.61) (width 0.6) (layer "F.Cu") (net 4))
 (segment (start 96.270798 71.013855) (end 97.485212 69.799441) (width 0.6) (layer "F.Cu") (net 3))
 (segment (start 110.49 68.315) (end 103.875 68.315) (width 0.6) (layer "F.Cu") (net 3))
 (segment (start 94.147966 71.577966) (end 95.28 72.71) (width 0.6) (layer "F.Cu") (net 3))
 (segment (start 99.06 63.5) (end 96.52 63.5) (width 0.6) (layer "F.Cu") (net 3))
 (segment (start 94.147966 71.013855) (end 96.270798 71.013855) (width 0.6) (layer "F.Cu") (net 3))
 (segment (start 96.52 63.5) (end 96.52 68.834229) (width 0.6) (layer "F.Cu") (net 3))
 (segment (start 103.875 68.315) (end 99.06 63.5) (width 0.6) (layer "F.Cu") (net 3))
 (segment (start 96.52 68.834229) (end 97.485212 69.799441) (width 0.6) (layer "F.Cu") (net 3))
 (segment (start 94.147966 71.013855) (end 94.147966 71.577966) (width 0.6) (layer "F.Cu") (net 3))
 (segment (start 121.24 79.883) (end 121.24 87.23) (width 0.6) (layer "F.Cu") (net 6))
 (segment (start 132.08 86.36) (end 125.45 86.36) (width 0.6) (layer "F.Cu") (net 6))
 (segment (start 121.24 87.23) (end 122.91 88.9) (width 0.6) (layer "F.Cu") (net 6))
 (segment (start 125.45 86.36) (end 122.91 88.9) (width 0.6) (layer "F.Cu") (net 6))
 (segment (start 121.24 77.597) (end 125.857 77.597) (width 0.6) (layer "F.Cu") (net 7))
 (segment (start 125.857 77.597) (end 132.08 83.82) (width 0.6) (layer "F.Cu") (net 7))
 (segment (start 123.19 74.93) (end 125.857 77.597) (width 0.6) (layer "F.Cu") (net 7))
 (segment (start 123.19 68.315) (end 123.19 74.93) (width 0.6) (layer "F.Cu") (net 7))
 (segment (start 127 66.04) (end 132.08 71.12) (width 0.6) (layer "F.Cu") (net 8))
 (segment (start 132.15 88.9) (end 134.62 86.43) (width 0.6) (layer "F.Cu") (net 8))
 (segment (start 134.62 86.43) (end 134.62 83.82) (width 0.6) (layer "F.Cu") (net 8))
 (segment (start 121.1525 67.8125) (end 122.925 66.04) (width 0.6) (layer "F.Cu") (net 8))
 (segment (start 122.925 66.04) (end 127 66.04) (width 0.6) (layer "F.Cu") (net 8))
 (segment (start 134.62 83.82) (end 132.08 81.28) (width 0.6) (layer "F.Cu") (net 8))
 (segment (start 120.65 68.315) (end 121.1525 67.8125) (width 0.6) (layer "F.Cu") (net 8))
 (segment (start 132.08 71.12) (end 132.08 81.28) (width 0.6) (layer "F.Cu") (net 8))
 (segment (start 126.01 88.9) (end 132.15 88.9) (width 0.6) (layer "F.Cu") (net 8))
 (segment (start 84.517822 120.077822) (end 95.085306 120.077822) (width 0.6) (layer "F.Cu") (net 9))
 (segment (start 99.06 70.83) (end 99.06 66.04) (width 0.6) (layer "F.Cu") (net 2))
 (segment (start 95.28 74.61) (end 99.06 70.83) (width 0.6) (layer "F.Cu") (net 2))
 (segment (start 95.085306 99.757822) (end 83.496054 99.757822) (width 0.6) (layer "F.Cu") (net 10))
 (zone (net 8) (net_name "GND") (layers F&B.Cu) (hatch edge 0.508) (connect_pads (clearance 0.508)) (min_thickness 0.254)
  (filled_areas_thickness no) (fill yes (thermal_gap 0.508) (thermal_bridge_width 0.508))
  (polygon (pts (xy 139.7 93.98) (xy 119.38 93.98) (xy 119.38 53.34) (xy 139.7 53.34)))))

